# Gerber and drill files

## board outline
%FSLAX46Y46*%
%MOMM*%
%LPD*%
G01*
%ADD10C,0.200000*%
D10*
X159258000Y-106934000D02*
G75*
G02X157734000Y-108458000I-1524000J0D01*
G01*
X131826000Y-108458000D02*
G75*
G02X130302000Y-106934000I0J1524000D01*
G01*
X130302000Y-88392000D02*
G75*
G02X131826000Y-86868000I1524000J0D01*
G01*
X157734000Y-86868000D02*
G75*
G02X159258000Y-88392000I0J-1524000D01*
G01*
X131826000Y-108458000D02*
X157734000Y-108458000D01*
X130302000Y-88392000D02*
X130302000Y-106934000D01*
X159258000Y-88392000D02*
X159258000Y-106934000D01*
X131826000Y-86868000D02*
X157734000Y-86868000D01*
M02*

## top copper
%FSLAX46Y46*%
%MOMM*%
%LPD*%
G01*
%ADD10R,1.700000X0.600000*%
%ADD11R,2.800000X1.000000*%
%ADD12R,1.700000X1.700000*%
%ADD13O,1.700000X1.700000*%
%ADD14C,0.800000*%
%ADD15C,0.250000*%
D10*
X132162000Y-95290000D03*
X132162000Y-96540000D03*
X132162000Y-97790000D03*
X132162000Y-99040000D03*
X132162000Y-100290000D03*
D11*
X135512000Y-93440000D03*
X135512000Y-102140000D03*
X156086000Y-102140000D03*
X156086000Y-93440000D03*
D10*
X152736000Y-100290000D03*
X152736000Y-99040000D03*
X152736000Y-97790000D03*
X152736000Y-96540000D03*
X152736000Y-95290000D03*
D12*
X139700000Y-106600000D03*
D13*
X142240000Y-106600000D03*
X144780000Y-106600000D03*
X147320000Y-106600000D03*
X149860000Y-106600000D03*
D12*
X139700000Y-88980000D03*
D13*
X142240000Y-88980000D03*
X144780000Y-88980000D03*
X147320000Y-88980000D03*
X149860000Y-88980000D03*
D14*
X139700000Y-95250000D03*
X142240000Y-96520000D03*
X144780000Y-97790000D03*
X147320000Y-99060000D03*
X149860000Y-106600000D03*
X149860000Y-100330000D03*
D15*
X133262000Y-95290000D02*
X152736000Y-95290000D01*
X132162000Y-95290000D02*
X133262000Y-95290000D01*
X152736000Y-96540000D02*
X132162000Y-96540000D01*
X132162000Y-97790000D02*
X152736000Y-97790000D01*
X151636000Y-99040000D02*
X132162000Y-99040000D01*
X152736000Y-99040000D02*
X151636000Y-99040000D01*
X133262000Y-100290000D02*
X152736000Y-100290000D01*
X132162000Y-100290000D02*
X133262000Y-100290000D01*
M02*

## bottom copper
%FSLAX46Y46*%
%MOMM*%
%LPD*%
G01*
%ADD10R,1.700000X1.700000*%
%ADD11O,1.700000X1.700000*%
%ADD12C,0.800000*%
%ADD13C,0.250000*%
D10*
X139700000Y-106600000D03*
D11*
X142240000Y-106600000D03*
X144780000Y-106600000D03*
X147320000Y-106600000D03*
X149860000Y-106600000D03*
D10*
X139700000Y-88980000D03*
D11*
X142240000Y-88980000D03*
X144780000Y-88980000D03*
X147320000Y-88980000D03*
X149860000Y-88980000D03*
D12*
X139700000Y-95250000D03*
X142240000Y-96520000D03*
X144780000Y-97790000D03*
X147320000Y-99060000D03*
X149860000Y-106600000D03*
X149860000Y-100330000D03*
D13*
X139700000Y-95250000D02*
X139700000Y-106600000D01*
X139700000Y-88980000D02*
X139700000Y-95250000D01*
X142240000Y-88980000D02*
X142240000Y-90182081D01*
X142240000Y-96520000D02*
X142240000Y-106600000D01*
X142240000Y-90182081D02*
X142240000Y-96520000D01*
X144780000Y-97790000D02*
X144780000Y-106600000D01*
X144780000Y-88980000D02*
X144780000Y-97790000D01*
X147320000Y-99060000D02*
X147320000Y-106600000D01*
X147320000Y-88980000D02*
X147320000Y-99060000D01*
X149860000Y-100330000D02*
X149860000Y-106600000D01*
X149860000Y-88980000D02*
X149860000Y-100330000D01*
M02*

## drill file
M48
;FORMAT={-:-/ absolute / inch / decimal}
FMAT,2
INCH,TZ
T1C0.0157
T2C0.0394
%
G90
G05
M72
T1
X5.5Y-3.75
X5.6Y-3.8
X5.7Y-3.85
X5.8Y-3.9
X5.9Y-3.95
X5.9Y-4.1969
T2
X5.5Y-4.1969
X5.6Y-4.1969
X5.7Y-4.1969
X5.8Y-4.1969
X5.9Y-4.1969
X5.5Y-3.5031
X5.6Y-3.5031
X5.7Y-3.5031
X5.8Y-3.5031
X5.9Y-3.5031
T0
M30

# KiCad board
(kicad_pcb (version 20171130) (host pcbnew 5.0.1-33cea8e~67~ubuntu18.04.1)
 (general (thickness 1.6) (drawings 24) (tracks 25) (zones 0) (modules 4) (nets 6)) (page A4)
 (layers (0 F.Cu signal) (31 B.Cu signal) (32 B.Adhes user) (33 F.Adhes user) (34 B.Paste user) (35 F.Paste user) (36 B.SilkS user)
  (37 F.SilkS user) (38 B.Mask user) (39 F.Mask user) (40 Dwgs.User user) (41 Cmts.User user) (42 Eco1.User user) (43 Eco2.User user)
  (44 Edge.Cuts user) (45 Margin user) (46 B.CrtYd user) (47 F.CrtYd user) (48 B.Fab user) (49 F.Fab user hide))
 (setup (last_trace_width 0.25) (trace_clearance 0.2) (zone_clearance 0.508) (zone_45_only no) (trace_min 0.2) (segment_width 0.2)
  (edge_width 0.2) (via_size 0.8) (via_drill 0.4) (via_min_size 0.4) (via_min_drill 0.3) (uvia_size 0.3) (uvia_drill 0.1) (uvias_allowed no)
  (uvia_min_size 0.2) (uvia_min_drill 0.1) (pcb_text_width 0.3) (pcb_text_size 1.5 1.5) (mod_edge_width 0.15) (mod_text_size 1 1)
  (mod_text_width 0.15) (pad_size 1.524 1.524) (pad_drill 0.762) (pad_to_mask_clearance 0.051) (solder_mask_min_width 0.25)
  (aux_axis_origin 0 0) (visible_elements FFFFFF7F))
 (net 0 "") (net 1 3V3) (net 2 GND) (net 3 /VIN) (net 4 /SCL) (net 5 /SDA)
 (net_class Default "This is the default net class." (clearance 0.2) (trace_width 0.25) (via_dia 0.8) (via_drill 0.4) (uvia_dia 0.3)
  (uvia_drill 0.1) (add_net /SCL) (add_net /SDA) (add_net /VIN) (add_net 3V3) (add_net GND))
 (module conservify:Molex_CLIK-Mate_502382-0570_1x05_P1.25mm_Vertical (layer F.Cu) (at 134.112 97.79 270)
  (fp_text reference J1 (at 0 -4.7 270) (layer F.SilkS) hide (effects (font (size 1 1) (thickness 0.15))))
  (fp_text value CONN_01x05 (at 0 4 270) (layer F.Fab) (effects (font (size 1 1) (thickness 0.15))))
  (pad 1 smd rect (at -2.5 1.95 270) (size 0.6 1.7) (layers F.Cu F.Paste F.Mask) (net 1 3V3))
  (pad 2 smd rect (at -1.25 1.95 270) (size 0.6 1.7) (layers F.Cu F.Paste F.Mask) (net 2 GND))
  (pad 3 smd rect (at 0 1.95 270) (size 0.6 1.7) (layers F.Cu F.Paste F.Mask) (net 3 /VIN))
  (pad 4 smd rect (at 1.25 1.95 270) (size 0.6 1.7) (layers F.Cu F.Paste F.Mask) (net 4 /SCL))
  (pad 5 smd rect (at 2.5 1.95 270) (size 0.6 1.7) (layers F.Cu F.Paste F.Mask) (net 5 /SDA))
  (pad "" smd rect (at -4.35 -1.4 270) (size 1 2.8) (layers F.Cu F.Paste F.Mask))
  (pad "" smd rect (at 4.35 -1.4 270) (size 1 2.8) (layers F.Cu F.Paste F.Mask)))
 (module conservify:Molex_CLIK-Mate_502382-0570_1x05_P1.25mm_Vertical (layer F.Cu) (at 154.686 97.79 270)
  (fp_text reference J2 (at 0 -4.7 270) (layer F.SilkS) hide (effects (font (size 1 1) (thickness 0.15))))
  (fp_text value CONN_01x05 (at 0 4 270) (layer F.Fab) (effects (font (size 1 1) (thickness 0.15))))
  (pad "" smd rect (at 4.35 -1.4 270) (size 1 2.8) (layers F.Cu F.Paste F.Mask))
  (pad "" smd rect (at -4.35 -1.4 270) (size 1 2.8) (layers F.Cu F.Paste F.Mask))
  (pad 5 smd rect (at 2.5 1.95 270) (size 0.6 1.7) (layers F.Cu F.Paste F.Mask) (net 5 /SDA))
  (pad 4 smd rect (at 1.25 1.95 270) (size 0.6 1.7) (layers F.Cu F.Paste F.Mask) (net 4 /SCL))
  (pad 3 smd rect (at 0 1.95 270) (size 0.6 1.7) (layers F.Cu F.Paste F.Mask) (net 3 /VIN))
  (pad 2 smd rect (at -1.25 1.95 270) (size 0.6 1.7) (layers F.Cu F.Paste F.Mask) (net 2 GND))
  (pad 1 smd rect (at -2.5 1.95 270) (size 0.6 1.7) (layers F.Cu F.Paste F.Mask) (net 1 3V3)))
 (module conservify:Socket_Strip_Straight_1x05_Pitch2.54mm (layer F.Cu) (at 139.7 106.6 90)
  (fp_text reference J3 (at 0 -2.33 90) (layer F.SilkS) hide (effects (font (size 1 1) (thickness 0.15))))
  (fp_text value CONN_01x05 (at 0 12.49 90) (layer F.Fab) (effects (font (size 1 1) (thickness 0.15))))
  (pad 1 thru_hole rect (at 0 0 90) (size 1.7 1.7) (drill 1) (layers *.Cu *.Mask) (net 1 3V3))
  (pad 2 thru_hole oval (at 0 2.54 90) (size 1.7 1.7) (drill 1) (layers *.Cu *.Mask) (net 2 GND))
  (pad 3 thru_hole oval (at 0 5.08 90) (size 1.7 1.7) (drill 1) (layers *.Cu *.Mask) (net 3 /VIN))
  (pad 4 thru_hole oval (at 0 7.62 90) (size 1.7 1.7) (drill 1) (layers *.Cu *.Mask) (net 4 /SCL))
  (pad 5 thru_hole oval (at 0 10.16 90) (size 1.7 1.7) (drill 1) (layers *.Cu *.Mask) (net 5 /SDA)))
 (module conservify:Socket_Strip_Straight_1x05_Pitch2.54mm (layer F.Cu) (at 139.7 88.98 90)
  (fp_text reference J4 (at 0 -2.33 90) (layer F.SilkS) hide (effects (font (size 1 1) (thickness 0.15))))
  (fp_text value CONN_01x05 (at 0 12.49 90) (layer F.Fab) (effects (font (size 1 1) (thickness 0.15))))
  (pad 1 thru_hole rect (at 0 0 90) (size 1.7 1.7) (drill 1) (layers *.Cu *.Mask) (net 1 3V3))
  (pad 2 thru_hole oval (at 0 2.54 90) (size 1.7 1.7) (drill 1) (layers *.Cu *.Mask) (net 2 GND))
  (pad 3 thru_hole oval (at 0 5.08 90) (size 1.7 1.7) (drill 1) (layers *.Cu *.Mask) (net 3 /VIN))
  (pad 4 thru_hole oval (at 0 7.62 90) (size 1.7 1.7) (drill 1) (layers *.Cu *.Mask) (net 4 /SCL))
  (pad 5 thru_hole oval (at 0 10.16 90) (size 1.7 1.7) (drill 1) (layers *.Cu *.Mask) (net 5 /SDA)))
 (gr_arc (start 157.734 106.934) (end 157.734 108.458) (angle -90) (layer Edge.Cuts) (width 0.2))
 (gr_arc (start 131.826 106.934) (end 130.302 106.934) (angle -90) (layer Edge.Cuts) (width 0.2))
 (gr_arc (start 131.826 88.392) (end 131.826 86.868) (angle -90) (layer Edge.Cuts) (width 0.2))
 (gr_arc (start 157.734 88.392) (end 159.258 88.392) (angle -90) (layer Edge.Cuts) (width 0.2))
 (gr_line (start 131.826 108.458) (end 157.734 108.458) (layer Edge.Cuts) (width 0.2))
 (gr_line (start 130.302 88.392) (end 130.302 106.934) (layer Edge.Cuts) (width 0.2))
 (gr_line (start 159.258 88.392) (end 159.258 106.934) (layer Edge.Cuts) (width 0.2))
 (gr_line (start 131.826 86.868) (end 157.734 86.868) (layer Edge.Cuts) (width 0.2))
 (segment (start 133.262 95.29) (end 152.736 95.29) (width 0.25) (layer F.Cu) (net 1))
 (segment (start 132.162 95.29) (end 133.262 95.29) (width 0.25) (layer F.Cu) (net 1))
 (via (at 139.7 95.25) (size 0.8) (drill 0.4) (layers F.Cu B.Cu) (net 1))
 (segment (start 139.7 95.25) (end 139.7 106.6) (width 0.25) (layer B.Cu) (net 1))
 (segment (start 139.7 88.98) (end 139.7 95.25) (width 0.25) (layer B.Cu) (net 1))
 (segment (start 152.736 96.54) (end 132.162 96.54) (width 0.25) (layer F.Cu) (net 2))
 (segment (start 142.24 88.98) (end 142.24 90.182081) (width 0.25) (layer B.Cu) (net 2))
 (via (at 142.24 96.52) (size 0.8) (drill 0.4) (layers F.Cu B.Cu) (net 2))
 (segment (start 142.24 96.52) (end 142.24 106.6) (width 0.25) (layer B.Cu) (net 2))
 (segment (start 142.24 90.182081) (end 142.24 96.52) (width 0.25) (layer B.Cu) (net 2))
 (segment (start 132.162 97.79) (end 152.736 97.79) (width 0.25) (layer F.Cu) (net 3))
 (via (at 144.78 97.79) (size 0.8) (drill 0.4) (layers F.Cu B.Cu) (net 3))
 (segment (start 144.78 97.79) (end 144.78 106.6) (width 0.25) (layer B.Cu) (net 3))
 (segment (start 144.78 88.98) (end 144.78 97.79) (width 0.25) (layer B.Cu) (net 3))
 (segment (start 151.636 99.04) (end 132.162 99.04) (width 0.25) (layer F.Cu) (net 4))
 (segment (start 152.736 99.04) (end 151.636 99.04) (width 0.25) (layer F.Cu) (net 4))
 (segment (start 147.32 99.06) (end 147.32 106.6) (width 0.25) (layer B.Cu) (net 4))
 (via (at 147.32 99.06) (size 0.8) (drill 0.4) (layers F.Cu B.Cu) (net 4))
 (segment (start 147.32 88.98) (end 147.32 99.06) (width 0.25) (layer B.Cu) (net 4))
 (segment (start 133.262 100.29) (end 152.736 100.29) (width 0.25) (layer F.Cu) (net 5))
 (segment (start 132.162 100.29) (end 133.262 100.29) (width 0.25) (layer F.Cu) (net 5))
 (via (at 149.86 106.6) (size 0.8) (drill 0.4) (layers F.Cu B.Cu) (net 5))
 (via (at 149.86 100.33) (size 0.8) (drill 0.4) (layers F.Cu B.Cu) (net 5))
 (segment (start 149.86 100.33) (end 149.86 106.6) (width 0.25) (layer B.Cu) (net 5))
 (segment (start 149.86 88.98) (end 149.86 100.33) (width 0.25) (layer B.Cu) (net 5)))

